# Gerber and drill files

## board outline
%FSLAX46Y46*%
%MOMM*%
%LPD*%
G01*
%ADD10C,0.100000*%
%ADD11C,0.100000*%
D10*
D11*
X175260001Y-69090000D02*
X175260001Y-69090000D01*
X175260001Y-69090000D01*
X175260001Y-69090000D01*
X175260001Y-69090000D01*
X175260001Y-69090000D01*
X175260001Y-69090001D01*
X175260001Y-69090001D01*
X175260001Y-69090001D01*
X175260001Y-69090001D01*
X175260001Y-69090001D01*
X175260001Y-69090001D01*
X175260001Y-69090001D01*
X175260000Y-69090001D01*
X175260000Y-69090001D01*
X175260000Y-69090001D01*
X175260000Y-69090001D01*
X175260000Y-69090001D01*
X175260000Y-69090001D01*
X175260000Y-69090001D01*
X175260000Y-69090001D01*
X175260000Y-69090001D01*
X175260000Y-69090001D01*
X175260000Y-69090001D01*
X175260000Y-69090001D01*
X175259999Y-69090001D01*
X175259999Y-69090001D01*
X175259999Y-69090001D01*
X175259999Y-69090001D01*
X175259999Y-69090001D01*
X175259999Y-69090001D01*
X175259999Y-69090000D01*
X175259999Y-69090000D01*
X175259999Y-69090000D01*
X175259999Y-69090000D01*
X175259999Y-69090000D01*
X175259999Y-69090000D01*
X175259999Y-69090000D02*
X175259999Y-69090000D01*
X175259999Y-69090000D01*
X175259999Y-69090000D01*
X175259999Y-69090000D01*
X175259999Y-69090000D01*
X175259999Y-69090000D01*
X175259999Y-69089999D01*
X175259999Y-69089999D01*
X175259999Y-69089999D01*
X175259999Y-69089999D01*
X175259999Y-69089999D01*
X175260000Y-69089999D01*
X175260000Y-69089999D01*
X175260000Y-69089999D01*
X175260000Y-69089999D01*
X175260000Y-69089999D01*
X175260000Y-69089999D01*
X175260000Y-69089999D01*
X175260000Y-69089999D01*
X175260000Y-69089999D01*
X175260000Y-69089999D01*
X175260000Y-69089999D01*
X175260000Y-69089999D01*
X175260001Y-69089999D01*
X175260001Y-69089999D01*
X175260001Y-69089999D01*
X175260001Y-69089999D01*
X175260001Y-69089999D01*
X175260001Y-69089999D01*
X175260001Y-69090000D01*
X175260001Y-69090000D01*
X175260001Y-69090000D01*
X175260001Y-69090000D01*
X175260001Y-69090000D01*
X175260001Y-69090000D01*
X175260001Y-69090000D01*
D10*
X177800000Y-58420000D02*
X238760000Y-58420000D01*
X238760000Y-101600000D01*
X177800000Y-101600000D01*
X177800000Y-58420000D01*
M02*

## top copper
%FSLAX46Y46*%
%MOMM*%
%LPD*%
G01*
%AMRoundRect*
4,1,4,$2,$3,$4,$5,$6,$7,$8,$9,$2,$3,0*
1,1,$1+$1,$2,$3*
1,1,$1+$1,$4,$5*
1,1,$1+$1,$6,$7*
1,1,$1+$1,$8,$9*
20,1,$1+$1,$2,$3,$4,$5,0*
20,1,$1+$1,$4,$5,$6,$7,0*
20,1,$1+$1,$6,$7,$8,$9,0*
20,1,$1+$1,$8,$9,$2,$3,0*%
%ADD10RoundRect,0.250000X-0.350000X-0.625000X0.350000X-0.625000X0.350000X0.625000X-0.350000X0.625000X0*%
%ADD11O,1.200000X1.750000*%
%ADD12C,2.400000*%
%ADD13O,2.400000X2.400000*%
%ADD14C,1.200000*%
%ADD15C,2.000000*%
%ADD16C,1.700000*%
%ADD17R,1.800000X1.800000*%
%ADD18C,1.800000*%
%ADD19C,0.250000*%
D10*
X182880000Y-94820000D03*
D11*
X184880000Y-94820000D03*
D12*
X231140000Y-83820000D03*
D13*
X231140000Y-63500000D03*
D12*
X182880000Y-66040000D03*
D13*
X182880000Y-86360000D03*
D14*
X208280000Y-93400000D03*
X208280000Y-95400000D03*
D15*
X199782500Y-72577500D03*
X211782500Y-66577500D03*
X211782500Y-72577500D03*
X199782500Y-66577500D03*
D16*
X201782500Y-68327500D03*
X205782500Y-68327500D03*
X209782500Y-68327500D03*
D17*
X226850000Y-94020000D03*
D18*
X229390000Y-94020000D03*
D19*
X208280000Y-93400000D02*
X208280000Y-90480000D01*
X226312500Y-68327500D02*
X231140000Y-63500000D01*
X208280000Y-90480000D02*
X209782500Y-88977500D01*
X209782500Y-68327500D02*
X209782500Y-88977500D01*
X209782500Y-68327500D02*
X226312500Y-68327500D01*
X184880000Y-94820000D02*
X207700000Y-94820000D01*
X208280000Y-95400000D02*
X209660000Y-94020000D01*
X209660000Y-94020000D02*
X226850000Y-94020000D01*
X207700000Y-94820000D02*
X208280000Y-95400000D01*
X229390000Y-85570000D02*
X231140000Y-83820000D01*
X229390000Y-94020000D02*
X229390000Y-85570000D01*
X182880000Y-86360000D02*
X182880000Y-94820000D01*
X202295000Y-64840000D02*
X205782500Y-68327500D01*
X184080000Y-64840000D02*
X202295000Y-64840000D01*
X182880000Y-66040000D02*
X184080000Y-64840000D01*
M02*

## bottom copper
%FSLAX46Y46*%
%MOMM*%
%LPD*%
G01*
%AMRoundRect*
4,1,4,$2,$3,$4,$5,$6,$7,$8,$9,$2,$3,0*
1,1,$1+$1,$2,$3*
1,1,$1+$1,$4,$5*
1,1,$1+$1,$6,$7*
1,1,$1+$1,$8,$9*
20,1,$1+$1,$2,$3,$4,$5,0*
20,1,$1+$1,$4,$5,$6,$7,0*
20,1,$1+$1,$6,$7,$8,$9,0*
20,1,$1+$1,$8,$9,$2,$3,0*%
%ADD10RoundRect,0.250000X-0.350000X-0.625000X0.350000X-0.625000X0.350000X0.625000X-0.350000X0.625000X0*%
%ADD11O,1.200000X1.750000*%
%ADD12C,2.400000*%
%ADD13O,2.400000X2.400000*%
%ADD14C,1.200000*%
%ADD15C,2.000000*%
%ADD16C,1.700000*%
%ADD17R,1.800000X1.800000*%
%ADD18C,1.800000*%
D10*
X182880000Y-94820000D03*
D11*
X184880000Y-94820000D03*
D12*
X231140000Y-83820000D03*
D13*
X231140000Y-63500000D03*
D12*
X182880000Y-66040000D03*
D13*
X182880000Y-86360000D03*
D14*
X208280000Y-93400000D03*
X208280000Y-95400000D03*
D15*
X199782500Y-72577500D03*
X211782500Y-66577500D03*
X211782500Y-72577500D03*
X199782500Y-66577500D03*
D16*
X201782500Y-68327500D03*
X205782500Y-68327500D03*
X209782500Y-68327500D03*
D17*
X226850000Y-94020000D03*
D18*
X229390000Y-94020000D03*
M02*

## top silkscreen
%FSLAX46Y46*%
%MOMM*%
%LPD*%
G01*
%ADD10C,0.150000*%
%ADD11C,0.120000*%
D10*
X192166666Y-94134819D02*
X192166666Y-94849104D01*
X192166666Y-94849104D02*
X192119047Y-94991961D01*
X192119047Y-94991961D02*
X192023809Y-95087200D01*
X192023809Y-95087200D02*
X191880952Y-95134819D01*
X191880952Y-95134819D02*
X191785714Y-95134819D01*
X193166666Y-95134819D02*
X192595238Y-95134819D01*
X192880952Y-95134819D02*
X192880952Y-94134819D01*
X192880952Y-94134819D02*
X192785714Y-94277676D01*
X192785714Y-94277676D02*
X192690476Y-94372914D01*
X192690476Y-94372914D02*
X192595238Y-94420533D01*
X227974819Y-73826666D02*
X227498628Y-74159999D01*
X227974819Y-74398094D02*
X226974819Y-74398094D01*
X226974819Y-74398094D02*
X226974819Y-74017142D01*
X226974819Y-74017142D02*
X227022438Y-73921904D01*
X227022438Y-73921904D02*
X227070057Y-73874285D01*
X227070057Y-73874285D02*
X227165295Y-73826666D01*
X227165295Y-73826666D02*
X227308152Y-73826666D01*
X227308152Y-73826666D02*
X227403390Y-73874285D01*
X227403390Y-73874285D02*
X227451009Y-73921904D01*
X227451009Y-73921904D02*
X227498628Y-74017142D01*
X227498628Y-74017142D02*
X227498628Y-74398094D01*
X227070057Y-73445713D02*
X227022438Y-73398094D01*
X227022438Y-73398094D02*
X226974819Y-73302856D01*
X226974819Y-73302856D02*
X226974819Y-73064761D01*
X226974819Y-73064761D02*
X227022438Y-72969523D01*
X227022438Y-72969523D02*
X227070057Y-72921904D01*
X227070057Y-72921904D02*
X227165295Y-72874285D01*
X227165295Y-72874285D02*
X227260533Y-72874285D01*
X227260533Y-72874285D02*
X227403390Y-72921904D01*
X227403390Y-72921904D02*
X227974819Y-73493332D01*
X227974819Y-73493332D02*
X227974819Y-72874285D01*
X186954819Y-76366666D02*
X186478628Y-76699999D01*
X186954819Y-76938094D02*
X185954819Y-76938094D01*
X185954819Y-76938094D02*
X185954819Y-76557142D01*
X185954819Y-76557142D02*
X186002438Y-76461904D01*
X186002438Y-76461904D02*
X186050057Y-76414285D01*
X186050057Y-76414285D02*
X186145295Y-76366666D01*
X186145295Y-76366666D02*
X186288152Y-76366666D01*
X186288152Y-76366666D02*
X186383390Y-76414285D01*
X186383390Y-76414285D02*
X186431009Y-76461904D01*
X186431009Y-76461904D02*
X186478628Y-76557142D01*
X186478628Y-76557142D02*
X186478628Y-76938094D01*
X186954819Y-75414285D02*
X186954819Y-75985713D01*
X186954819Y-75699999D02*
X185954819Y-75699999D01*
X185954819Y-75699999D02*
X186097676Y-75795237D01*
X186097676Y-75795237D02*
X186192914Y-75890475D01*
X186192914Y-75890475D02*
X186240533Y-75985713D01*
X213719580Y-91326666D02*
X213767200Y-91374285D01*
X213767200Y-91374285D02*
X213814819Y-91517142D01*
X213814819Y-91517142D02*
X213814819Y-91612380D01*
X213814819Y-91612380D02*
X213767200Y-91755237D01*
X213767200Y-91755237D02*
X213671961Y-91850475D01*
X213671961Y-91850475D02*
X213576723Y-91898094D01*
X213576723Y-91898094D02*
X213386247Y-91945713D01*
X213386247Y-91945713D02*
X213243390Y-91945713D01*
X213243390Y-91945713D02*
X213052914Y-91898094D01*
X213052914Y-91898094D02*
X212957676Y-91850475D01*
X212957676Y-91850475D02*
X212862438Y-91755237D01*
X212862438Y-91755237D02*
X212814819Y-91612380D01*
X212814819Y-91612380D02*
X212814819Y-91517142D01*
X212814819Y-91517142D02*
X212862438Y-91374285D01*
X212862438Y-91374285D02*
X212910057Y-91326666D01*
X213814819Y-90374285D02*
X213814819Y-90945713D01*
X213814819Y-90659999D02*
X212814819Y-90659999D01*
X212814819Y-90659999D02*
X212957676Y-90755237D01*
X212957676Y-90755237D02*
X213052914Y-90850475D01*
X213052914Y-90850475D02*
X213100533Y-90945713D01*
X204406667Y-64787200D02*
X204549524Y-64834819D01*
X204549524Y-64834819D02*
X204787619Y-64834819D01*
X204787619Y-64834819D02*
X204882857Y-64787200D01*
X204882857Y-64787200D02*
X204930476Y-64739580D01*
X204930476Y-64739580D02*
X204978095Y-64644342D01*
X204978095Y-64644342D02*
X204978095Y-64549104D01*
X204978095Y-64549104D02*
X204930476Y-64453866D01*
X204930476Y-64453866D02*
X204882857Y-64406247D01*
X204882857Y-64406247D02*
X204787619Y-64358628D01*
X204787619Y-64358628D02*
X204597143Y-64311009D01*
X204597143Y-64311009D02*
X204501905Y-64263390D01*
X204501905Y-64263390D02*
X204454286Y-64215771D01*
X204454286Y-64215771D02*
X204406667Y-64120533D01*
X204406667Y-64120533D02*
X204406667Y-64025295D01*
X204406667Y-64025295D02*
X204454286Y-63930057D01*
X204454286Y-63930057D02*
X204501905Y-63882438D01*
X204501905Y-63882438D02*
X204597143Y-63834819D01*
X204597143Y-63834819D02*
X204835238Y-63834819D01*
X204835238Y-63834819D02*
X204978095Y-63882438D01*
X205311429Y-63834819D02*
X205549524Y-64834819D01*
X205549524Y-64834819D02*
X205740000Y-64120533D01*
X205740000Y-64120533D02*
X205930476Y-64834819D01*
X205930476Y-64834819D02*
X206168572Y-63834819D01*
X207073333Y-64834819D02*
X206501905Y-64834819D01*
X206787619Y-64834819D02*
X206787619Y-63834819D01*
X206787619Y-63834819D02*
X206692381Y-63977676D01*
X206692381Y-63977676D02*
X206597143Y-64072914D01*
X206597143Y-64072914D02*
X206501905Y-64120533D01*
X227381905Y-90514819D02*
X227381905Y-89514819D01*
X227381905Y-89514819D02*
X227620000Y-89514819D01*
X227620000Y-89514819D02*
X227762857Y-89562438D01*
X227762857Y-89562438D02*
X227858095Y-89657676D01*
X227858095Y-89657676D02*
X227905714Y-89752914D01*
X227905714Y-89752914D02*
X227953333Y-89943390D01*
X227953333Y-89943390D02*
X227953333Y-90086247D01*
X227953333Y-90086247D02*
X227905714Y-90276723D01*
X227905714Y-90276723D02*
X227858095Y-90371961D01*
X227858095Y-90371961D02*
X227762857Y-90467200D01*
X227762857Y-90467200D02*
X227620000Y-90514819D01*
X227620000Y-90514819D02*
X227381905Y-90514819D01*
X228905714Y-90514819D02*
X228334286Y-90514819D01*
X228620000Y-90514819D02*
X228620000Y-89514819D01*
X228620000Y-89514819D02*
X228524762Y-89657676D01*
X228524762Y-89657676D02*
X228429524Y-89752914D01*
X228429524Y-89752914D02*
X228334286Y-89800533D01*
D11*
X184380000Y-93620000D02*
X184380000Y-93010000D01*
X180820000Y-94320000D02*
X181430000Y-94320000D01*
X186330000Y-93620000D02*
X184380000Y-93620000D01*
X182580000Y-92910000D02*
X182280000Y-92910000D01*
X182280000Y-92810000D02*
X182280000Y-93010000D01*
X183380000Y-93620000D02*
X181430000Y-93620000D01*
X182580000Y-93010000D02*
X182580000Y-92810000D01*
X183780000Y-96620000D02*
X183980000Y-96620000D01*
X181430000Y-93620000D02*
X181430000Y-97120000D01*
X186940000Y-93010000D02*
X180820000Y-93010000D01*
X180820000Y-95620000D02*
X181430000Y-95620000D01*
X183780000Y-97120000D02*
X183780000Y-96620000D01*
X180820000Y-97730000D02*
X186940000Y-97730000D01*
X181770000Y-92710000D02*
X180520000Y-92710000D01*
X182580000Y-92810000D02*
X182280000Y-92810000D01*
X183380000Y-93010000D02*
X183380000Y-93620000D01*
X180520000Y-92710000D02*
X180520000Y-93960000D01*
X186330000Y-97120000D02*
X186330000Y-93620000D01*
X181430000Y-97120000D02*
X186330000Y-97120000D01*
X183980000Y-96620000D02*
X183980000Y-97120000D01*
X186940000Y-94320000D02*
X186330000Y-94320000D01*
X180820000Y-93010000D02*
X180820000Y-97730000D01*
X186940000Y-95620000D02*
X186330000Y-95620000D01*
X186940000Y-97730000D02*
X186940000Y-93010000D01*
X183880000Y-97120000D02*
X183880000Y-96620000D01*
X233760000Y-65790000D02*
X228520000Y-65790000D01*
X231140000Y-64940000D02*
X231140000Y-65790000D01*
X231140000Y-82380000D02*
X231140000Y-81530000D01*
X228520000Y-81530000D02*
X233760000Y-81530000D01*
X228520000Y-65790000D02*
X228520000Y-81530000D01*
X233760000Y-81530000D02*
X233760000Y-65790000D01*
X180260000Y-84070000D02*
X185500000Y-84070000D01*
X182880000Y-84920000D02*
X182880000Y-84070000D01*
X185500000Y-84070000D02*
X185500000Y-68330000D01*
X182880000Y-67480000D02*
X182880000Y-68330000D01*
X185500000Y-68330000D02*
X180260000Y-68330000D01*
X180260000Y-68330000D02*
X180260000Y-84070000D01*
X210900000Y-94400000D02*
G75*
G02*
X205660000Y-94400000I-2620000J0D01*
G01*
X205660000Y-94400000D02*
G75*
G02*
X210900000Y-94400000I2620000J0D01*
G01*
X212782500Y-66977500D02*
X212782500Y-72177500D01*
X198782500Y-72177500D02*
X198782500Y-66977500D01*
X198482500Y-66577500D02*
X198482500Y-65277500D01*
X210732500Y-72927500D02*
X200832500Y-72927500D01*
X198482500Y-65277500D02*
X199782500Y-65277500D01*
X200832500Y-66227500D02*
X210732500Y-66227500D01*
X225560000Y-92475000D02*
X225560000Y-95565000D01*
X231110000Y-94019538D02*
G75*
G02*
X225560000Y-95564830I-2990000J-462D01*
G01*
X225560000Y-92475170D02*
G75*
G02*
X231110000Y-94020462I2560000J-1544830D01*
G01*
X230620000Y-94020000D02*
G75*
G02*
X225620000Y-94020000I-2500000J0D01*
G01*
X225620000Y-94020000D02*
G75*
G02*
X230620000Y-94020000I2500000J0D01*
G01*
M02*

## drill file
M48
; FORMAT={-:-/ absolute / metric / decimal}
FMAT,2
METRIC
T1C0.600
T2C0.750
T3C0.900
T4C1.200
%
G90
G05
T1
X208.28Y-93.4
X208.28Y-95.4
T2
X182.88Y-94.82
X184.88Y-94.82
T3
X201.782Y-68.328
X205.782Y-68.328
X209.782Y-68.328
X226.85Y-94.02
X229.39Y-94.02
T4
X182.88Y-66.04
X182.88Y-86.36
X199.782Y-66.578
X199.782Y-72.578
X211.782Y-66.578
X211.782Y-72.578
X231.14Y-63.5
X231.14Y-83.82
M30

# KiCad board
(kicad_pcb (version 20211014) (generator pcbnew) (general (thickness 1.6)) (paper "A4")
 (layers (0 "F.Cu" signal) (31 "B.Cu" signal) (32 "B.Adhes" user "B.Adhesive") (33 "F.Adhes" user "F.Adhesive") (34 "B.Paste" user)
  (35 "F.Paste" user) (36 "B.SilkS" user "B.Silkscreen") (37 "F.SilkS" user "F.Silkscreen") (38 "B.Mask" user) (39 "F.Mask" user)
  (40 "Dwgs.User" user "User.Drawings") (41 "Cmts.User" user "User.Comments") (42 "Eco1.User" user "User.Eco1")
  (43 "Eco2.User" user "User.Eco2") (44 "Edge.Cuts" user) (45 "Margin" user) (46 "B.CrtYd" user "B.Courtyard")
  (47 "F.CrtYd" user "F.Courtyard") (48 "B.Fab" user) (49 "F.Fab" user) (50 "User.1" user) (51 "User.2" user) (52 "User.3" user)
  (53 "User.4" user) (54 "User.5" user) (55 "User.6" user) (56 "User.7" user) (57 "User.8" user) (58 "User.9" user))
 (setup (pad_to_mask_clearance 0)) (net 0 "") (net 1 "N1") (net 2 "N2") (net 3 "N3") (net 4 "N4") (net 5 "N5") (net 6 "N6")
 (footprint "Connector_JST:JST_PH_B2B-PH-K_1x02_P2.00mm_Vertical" (layer "F.Cu") (at 182.88 94.82)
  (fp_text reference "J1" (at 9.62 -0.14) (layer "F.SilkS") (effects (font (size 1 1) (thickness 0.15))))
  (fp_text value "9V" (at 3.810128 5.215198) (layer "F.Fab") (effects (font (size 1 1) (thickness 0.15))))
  (fp_line (start 1.5 -1.2) (end 1.5 -1.81) (layer "F.SilkS") (width 0.12))
  (fp_line (start -2.06 -0.5) (end -1.45 -0.5) (layer "F.SilkS") (width 0.12))
  (fp_line (start 3.45 -1.2) (end 1.5 -1.2) (layer "F.SilkS") (width 0.12))
  (fp_line (start -0.3 -1.91) (end -0.6 -1.91) (layer "F.SilkS") (width 0.12))
  (fp_line (start -0.6 -2.01) (end -0.6 -1.81) (layer "F.SilkS") (width 0.12))
  (fp_line (start 0.5 -1.2) (end -1.45 -1.2) (layer "F.SilkS") (width 0.12))
  (fp_line (start -0.3 -1.81) (end -0.3 -2.01) (layer "F.SilkS") (width 0.12))
  (fp_line (start 0.9 1.8) (end 1.1 1.8) (layer "F.SilkS") (width 0.12))
  (fp_line (start -1.45 -1.2) (end -1.45 2.3) (layer "F.SilkS") (width 0.12))
  (fp_line (start 4.06 -1.81) (end -2.06 -1.81) (layer "F.SilkS") (width 0.12))
  (fp_line (start -2.06 0.8) (end -1.45 0.8) (layer "F.SilkS") (width 0.12))
  (fp_line (start 0.9 2.3) (end 0.9 1.8) (layer "F.SilkS") (width 0.12))
  (fp_line (start -2.06 2.91) (end 4.06 2.91) (layer "F.SilkS") (width 0.12))
  (fp_line (start -1.11 -2.11) (end -2.36 -2.11) (layer "F.SilkS") (width 0.12))
  (fp_line (start -0.3 -2.01) (end -0.6 -2.01) (layer "F.SilkS") (width 0.12))
  (fp_line (start 0.5 -1.81) (end 0.5 -1.2) (layer "F.SilkS") (width 0.12))
  (fp_line (start -2.36 -2.11) (end -2.36 -0.86) (layer "F.SilkS") (width 0.12))
  (fp_line (start 3.45 2.3) (end 3.45 -1.2) (layer "F.SilkS") (width 0.12))
  (fp_line (start -1.45 2.3) (end 3.45 2.3) (layer "F.SilkS") (width 0.12))
  (fp_line (start 1.1 1.8) (end 1.1 2.3) (layer "F.SilkS") (width 0.12))
  (fp_line (start 4.06 -0.5) (end 3.45 -0.5) (layer "F.SilkS") (width 0.12))
  (fp_line (start -2.06 -1.81) (end -2.06 2.91) (layer "F.SilkS") (width 0.12))
  (fp_line (start 4.06 0.8) (end 3.45 0.8) (layer "F.SilkS") (width 0.12))
  (fp_line (start 4.06 2.91) (end 4.06 -1.81) (layer "F.SilkS") (width 0.12))
  (fp_line (start 1 2.3) (end 1 1.8) (layer "F.SilkS") (width 0.12))
  (pad "1" thru_hole roundrect (at 0 0) (size 1.2 1.75) (drill 0.75) (layers *.Cu *.Mask) (roundrect_rratio 0.208333) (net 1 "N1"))
  (pad "2" thru_hole oval (at 2 0) (size 1.2 1.75) (drill 0.75) (layers *.Cu *.Mask) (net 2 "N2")))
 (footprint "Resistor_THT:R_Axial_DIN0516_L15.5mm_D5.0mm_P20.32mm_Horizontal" (layer "F.Cu") (at 231.14 83.82 90)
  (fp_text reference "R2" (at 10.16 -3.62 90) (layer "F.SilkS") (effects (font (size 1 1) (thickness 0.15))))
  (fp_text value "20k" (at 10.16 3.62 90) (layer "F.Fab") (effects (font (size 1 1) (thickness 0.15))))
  (fp_line (start 18.03 2.62) (end 18.03 -2.62) (layer "F.SilkS") (width 0.12))
  (fp_line (start 18.88 0) (end 18.03 0) (layer "F.SilkS") (width 0.12))
  (fp_line (start 1.44 0) (end 2.29 0) (layer "F.SilkS") (width 0.12))
  (fp_line (start 2.29 -2.62) (end 2.29 2.62) (layer "F.SilkS") (width 0.12))
  (fp_line (start 18.03 -2.62) (end 2.29 -2.62) (layer "F.SilkS") (width 0.12))
  (fp_line (start 2.29 2.62) (end 18.03 2.62) (layer "F.SilkS") (width 0.12))
  (pad "1" thru_hole circle (at 0 0 90) (size 2.4 2.4) (drill 1.2) (layers *.Cu *.Mask) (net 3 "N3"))
  (pad "2" thru_hole oval (at 20.32 0 90) (size 2.4 2.4) (drill 1.2) (layers *.Cu *.Mask) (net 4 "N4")))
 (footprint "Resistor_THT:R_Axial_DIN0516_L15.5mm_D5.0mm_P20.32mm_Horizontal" (layer "F.Cu") (at 182.88 66.04 -90)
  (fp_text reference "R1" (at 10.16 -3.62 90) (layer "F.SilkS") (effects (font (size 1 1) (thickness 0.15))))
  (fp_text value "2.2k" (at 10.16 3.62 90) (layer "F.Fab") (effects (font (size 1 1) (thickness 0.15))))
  (fp_line (start 18.03 2.62) (end 18.03 -2.62) (layer "F.SilkS") (width 0.12))
  (fp_line (start 18.88 0) (end 18.03 0) (layer "F.SilkS") (width 0.12))
  (fp_line (start 18.03 -2.62) (end 2.29 -2.62) (layer "F.SilkS") (width 0.12))
  (fp_line (start 1.44 0) (end 2.29 0) (layer "F.SilkS") (width 0.12))
  (fp_line (start 2.29 -2.62) (end 2.29 2.62) (layer "F.SilkS") (width 0.12))
  (fp_line (start 2.29 2.62) (end 18.03 2.62) (layer "F.SilkS") (width 0.12))
  (pad "1" thru_hole circle (at 0 0 270) (size 2.4 2.4) (drill 1.2) (layers *.Cu *.Mask) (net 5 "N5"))
  (pad "2" thru_hole oval (at 20.32 0 270) (size 2.4 2.4) (drill 1.2) (layers *.Cu *.Mask) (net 1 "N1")))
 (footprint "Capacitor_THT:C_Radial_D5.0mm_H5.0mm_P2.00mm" (layer "F.Cu") (at 208.28 93.4 -90)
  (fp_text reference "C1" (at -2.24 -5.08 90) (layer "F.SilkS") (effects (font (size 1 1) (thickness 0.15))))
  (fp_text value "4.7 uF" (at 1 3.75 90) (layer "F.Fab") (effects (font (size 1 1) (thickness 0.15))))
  (fp_circle (center 1 0) (end 3.62 0) (layer "F.SilkS") (width 0.12) (fill none))
  (pad "1" thru_hole circle (at 0 0 270) (size 1.2 1.2) (drill 0.6) (layers *.Cu *.Mask) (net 4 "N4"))
  (pad "2" thru_hole circle (at 2 0 270) (size 1.2 1.2) (drill 0.6) (layers *.Cu *.Mask) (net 2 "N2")))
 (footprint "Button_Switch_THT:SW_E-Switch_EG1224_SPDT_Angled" (layer "F.Cu") (at 201.7825 68.3275)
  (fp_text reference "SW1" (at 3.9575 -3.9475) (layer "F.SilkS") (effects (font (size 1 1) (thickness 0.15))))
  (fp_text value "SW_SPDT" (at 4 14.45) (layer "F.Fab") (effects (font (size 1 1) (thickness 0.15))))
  (fp_line (start 11 -1.35) (end 11 3.85) (layer "F.SilkS") (width 0.12))
  (fp_line (start -3 3.85) (end -3 -1.35) (layer "F.SilkS") (width 0.12))
  (fp_line (start -3.3 -1.75) (end -3.3 -3.05) (layer "F.SilkS") (width 0.12))
  (fp_line (start 8.95 4.6) (end -0.95 4.6) (layer "F.SilkS") (width 0.12))
  (fp_line (start -3.3 -3.05) (end -2 -3.05) (layer "F.SilkS") (width 0.12))
  (fp_line (start -0.95 -2.1) (end 8.95 -2.1) (layer "F.SilkS") (width 0.12))
  (pad "" thru_hole circle (at -2 4.25) (size 2 2) (drill 1.2) (layers *.Cu *.Mask))
  (pad "" thru_hole circle (at 10 -1.75) (size 2 2) (drill 1.2) (layers *.Cu *.Mask))
  (pad "" thru_hole circle (at 10 4.25) (size 2 2) (drill 1.2) (layers *.Cu *.Mask))
  (pad "" thru_hole circle (at -2 -1.75) (size 2 2) (drill 1.2) (layers *.Cu *.Mask))
  (pad "1" thru_hole circle (at 0 0) (size 1.7 1.7) (drill 0.9) (layers *.Cu *.Mask) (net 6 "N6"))
  (pad "2" thru_hole circle (at 4 0) (size 1.7 1.7) (drill 0.9) (layers *.Cu *.Mask) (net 5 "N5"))
  (pad "3" thru_hole circle (at 8 0) (size 1.7 1.7) (drill 0.9) (layers *.Cu *.Mask) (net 4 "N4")))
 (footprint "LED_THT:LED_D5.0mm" (layer "F.Cu") (at 226.85 94.02)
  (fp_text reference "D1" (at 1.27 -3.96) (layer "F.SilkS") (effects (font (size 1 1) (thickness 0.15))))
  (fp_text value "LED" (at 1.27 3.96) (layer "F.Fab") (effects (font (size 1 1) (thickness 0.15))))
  (fp_line (start -1.29 -1.545) (end -1.29 1.545) (layer "F.SilkS") (width 0.12))
  (fp_arc (start 4.26 -0.000462) (mid 2.072002 2.880433) (end -1.29 1.54483) (layer "F.SilkS") (width 0.12))
  (fp_arc (start -1.29 -1.54483) (mid 2.072002 -2.880433) (end 4.26 0.000462) (layer "F.SilkS") (width 0.12))
  (fp_circle (center 1.27 0) (end 3.77 0) (layer "F.SilkS") (width 0.12) (fill none))
  (pad "1" thru_hole rect (at 0 0) (size 1.8 1.8) (drill 0.9) (layers *.Cu *.Mask) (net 2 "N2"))
  (pad "2" thru_hole circle (at 2.54 0) (size 1.8 1.8) (drill 0.9) (layers *.Cu *.Mask) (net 3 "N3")))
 (gr_circle (center 175.26 69.09) (end 175.26 69.09) (layer "Edge.Cuts") (width 0.1) (fill none))
 (gr_rect (start 177.8 58.42) (end 238.76 101.6) (layer "Edge.Cuts") (width 0.1) (fill none))
 (segment (start 208.28 93.4) (end 208.28 90.48) (width 0.25) (layer "F.Cu") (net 4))
 (segment (start 226.3125 68.3275) (end 231.14 63.5) (width 0.25) (layer "F.Cu") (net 4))
 (segment (start 208.28 90.48) (end 209.7825 88.9775) (width 0.25) (layer "F.Cu") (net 4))
 (segment (start 209.7825 68.3275) (end 209.7825 88.9775) (width 0.25) (layer "F.Cu") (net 4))
 (segment (start 209.7825 68.3275) (end 226.3125 68.3275) (width 0.25) (layer "F.Cu") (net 4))
 (segment (start 184.88 94.82) (end 207.7 94.82) (width 0.25) (layer "F.Cu") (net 2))
 (segment (start 208.28 95.4) (end 209.66 94.02) (width 0.25) (layer "F.Cu") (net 2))
 (segment (start 209.66 94.02) (end 226.85 94.02) (width 0.25) (layer "F.Cu") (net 2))
 (segment (start 207.7 94.82) (end 208.28 95.4) (width 0.25) (layer "F.Cu") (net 2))
 (segment (start 229.39 85.57) (end 231.14 83.82) (width 0.25) (layer "F.Cu") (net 3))
 (segment (start 229.39 94.02) (end 229.39 85.57) (width 0.25) (layer "F.Cu") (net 3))
 (segment (start 182.88 86.36) (end 182.88 94.82) (width 0.25) (layer "F.Cu") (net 1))
 (segment (start 202.295 64.84) (end 205.7825 68.3275) (width 0.25) (layer "F.Cu") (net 5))
 (segment (start 184.08 64.84) (end 202.295 64.84) (width 0.25) (layer "F.Cu") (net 5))
 (segment (start 182.88 66.04) (end 184.08 64.84) (width 0.25) (layer "F.Cu") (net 5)))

